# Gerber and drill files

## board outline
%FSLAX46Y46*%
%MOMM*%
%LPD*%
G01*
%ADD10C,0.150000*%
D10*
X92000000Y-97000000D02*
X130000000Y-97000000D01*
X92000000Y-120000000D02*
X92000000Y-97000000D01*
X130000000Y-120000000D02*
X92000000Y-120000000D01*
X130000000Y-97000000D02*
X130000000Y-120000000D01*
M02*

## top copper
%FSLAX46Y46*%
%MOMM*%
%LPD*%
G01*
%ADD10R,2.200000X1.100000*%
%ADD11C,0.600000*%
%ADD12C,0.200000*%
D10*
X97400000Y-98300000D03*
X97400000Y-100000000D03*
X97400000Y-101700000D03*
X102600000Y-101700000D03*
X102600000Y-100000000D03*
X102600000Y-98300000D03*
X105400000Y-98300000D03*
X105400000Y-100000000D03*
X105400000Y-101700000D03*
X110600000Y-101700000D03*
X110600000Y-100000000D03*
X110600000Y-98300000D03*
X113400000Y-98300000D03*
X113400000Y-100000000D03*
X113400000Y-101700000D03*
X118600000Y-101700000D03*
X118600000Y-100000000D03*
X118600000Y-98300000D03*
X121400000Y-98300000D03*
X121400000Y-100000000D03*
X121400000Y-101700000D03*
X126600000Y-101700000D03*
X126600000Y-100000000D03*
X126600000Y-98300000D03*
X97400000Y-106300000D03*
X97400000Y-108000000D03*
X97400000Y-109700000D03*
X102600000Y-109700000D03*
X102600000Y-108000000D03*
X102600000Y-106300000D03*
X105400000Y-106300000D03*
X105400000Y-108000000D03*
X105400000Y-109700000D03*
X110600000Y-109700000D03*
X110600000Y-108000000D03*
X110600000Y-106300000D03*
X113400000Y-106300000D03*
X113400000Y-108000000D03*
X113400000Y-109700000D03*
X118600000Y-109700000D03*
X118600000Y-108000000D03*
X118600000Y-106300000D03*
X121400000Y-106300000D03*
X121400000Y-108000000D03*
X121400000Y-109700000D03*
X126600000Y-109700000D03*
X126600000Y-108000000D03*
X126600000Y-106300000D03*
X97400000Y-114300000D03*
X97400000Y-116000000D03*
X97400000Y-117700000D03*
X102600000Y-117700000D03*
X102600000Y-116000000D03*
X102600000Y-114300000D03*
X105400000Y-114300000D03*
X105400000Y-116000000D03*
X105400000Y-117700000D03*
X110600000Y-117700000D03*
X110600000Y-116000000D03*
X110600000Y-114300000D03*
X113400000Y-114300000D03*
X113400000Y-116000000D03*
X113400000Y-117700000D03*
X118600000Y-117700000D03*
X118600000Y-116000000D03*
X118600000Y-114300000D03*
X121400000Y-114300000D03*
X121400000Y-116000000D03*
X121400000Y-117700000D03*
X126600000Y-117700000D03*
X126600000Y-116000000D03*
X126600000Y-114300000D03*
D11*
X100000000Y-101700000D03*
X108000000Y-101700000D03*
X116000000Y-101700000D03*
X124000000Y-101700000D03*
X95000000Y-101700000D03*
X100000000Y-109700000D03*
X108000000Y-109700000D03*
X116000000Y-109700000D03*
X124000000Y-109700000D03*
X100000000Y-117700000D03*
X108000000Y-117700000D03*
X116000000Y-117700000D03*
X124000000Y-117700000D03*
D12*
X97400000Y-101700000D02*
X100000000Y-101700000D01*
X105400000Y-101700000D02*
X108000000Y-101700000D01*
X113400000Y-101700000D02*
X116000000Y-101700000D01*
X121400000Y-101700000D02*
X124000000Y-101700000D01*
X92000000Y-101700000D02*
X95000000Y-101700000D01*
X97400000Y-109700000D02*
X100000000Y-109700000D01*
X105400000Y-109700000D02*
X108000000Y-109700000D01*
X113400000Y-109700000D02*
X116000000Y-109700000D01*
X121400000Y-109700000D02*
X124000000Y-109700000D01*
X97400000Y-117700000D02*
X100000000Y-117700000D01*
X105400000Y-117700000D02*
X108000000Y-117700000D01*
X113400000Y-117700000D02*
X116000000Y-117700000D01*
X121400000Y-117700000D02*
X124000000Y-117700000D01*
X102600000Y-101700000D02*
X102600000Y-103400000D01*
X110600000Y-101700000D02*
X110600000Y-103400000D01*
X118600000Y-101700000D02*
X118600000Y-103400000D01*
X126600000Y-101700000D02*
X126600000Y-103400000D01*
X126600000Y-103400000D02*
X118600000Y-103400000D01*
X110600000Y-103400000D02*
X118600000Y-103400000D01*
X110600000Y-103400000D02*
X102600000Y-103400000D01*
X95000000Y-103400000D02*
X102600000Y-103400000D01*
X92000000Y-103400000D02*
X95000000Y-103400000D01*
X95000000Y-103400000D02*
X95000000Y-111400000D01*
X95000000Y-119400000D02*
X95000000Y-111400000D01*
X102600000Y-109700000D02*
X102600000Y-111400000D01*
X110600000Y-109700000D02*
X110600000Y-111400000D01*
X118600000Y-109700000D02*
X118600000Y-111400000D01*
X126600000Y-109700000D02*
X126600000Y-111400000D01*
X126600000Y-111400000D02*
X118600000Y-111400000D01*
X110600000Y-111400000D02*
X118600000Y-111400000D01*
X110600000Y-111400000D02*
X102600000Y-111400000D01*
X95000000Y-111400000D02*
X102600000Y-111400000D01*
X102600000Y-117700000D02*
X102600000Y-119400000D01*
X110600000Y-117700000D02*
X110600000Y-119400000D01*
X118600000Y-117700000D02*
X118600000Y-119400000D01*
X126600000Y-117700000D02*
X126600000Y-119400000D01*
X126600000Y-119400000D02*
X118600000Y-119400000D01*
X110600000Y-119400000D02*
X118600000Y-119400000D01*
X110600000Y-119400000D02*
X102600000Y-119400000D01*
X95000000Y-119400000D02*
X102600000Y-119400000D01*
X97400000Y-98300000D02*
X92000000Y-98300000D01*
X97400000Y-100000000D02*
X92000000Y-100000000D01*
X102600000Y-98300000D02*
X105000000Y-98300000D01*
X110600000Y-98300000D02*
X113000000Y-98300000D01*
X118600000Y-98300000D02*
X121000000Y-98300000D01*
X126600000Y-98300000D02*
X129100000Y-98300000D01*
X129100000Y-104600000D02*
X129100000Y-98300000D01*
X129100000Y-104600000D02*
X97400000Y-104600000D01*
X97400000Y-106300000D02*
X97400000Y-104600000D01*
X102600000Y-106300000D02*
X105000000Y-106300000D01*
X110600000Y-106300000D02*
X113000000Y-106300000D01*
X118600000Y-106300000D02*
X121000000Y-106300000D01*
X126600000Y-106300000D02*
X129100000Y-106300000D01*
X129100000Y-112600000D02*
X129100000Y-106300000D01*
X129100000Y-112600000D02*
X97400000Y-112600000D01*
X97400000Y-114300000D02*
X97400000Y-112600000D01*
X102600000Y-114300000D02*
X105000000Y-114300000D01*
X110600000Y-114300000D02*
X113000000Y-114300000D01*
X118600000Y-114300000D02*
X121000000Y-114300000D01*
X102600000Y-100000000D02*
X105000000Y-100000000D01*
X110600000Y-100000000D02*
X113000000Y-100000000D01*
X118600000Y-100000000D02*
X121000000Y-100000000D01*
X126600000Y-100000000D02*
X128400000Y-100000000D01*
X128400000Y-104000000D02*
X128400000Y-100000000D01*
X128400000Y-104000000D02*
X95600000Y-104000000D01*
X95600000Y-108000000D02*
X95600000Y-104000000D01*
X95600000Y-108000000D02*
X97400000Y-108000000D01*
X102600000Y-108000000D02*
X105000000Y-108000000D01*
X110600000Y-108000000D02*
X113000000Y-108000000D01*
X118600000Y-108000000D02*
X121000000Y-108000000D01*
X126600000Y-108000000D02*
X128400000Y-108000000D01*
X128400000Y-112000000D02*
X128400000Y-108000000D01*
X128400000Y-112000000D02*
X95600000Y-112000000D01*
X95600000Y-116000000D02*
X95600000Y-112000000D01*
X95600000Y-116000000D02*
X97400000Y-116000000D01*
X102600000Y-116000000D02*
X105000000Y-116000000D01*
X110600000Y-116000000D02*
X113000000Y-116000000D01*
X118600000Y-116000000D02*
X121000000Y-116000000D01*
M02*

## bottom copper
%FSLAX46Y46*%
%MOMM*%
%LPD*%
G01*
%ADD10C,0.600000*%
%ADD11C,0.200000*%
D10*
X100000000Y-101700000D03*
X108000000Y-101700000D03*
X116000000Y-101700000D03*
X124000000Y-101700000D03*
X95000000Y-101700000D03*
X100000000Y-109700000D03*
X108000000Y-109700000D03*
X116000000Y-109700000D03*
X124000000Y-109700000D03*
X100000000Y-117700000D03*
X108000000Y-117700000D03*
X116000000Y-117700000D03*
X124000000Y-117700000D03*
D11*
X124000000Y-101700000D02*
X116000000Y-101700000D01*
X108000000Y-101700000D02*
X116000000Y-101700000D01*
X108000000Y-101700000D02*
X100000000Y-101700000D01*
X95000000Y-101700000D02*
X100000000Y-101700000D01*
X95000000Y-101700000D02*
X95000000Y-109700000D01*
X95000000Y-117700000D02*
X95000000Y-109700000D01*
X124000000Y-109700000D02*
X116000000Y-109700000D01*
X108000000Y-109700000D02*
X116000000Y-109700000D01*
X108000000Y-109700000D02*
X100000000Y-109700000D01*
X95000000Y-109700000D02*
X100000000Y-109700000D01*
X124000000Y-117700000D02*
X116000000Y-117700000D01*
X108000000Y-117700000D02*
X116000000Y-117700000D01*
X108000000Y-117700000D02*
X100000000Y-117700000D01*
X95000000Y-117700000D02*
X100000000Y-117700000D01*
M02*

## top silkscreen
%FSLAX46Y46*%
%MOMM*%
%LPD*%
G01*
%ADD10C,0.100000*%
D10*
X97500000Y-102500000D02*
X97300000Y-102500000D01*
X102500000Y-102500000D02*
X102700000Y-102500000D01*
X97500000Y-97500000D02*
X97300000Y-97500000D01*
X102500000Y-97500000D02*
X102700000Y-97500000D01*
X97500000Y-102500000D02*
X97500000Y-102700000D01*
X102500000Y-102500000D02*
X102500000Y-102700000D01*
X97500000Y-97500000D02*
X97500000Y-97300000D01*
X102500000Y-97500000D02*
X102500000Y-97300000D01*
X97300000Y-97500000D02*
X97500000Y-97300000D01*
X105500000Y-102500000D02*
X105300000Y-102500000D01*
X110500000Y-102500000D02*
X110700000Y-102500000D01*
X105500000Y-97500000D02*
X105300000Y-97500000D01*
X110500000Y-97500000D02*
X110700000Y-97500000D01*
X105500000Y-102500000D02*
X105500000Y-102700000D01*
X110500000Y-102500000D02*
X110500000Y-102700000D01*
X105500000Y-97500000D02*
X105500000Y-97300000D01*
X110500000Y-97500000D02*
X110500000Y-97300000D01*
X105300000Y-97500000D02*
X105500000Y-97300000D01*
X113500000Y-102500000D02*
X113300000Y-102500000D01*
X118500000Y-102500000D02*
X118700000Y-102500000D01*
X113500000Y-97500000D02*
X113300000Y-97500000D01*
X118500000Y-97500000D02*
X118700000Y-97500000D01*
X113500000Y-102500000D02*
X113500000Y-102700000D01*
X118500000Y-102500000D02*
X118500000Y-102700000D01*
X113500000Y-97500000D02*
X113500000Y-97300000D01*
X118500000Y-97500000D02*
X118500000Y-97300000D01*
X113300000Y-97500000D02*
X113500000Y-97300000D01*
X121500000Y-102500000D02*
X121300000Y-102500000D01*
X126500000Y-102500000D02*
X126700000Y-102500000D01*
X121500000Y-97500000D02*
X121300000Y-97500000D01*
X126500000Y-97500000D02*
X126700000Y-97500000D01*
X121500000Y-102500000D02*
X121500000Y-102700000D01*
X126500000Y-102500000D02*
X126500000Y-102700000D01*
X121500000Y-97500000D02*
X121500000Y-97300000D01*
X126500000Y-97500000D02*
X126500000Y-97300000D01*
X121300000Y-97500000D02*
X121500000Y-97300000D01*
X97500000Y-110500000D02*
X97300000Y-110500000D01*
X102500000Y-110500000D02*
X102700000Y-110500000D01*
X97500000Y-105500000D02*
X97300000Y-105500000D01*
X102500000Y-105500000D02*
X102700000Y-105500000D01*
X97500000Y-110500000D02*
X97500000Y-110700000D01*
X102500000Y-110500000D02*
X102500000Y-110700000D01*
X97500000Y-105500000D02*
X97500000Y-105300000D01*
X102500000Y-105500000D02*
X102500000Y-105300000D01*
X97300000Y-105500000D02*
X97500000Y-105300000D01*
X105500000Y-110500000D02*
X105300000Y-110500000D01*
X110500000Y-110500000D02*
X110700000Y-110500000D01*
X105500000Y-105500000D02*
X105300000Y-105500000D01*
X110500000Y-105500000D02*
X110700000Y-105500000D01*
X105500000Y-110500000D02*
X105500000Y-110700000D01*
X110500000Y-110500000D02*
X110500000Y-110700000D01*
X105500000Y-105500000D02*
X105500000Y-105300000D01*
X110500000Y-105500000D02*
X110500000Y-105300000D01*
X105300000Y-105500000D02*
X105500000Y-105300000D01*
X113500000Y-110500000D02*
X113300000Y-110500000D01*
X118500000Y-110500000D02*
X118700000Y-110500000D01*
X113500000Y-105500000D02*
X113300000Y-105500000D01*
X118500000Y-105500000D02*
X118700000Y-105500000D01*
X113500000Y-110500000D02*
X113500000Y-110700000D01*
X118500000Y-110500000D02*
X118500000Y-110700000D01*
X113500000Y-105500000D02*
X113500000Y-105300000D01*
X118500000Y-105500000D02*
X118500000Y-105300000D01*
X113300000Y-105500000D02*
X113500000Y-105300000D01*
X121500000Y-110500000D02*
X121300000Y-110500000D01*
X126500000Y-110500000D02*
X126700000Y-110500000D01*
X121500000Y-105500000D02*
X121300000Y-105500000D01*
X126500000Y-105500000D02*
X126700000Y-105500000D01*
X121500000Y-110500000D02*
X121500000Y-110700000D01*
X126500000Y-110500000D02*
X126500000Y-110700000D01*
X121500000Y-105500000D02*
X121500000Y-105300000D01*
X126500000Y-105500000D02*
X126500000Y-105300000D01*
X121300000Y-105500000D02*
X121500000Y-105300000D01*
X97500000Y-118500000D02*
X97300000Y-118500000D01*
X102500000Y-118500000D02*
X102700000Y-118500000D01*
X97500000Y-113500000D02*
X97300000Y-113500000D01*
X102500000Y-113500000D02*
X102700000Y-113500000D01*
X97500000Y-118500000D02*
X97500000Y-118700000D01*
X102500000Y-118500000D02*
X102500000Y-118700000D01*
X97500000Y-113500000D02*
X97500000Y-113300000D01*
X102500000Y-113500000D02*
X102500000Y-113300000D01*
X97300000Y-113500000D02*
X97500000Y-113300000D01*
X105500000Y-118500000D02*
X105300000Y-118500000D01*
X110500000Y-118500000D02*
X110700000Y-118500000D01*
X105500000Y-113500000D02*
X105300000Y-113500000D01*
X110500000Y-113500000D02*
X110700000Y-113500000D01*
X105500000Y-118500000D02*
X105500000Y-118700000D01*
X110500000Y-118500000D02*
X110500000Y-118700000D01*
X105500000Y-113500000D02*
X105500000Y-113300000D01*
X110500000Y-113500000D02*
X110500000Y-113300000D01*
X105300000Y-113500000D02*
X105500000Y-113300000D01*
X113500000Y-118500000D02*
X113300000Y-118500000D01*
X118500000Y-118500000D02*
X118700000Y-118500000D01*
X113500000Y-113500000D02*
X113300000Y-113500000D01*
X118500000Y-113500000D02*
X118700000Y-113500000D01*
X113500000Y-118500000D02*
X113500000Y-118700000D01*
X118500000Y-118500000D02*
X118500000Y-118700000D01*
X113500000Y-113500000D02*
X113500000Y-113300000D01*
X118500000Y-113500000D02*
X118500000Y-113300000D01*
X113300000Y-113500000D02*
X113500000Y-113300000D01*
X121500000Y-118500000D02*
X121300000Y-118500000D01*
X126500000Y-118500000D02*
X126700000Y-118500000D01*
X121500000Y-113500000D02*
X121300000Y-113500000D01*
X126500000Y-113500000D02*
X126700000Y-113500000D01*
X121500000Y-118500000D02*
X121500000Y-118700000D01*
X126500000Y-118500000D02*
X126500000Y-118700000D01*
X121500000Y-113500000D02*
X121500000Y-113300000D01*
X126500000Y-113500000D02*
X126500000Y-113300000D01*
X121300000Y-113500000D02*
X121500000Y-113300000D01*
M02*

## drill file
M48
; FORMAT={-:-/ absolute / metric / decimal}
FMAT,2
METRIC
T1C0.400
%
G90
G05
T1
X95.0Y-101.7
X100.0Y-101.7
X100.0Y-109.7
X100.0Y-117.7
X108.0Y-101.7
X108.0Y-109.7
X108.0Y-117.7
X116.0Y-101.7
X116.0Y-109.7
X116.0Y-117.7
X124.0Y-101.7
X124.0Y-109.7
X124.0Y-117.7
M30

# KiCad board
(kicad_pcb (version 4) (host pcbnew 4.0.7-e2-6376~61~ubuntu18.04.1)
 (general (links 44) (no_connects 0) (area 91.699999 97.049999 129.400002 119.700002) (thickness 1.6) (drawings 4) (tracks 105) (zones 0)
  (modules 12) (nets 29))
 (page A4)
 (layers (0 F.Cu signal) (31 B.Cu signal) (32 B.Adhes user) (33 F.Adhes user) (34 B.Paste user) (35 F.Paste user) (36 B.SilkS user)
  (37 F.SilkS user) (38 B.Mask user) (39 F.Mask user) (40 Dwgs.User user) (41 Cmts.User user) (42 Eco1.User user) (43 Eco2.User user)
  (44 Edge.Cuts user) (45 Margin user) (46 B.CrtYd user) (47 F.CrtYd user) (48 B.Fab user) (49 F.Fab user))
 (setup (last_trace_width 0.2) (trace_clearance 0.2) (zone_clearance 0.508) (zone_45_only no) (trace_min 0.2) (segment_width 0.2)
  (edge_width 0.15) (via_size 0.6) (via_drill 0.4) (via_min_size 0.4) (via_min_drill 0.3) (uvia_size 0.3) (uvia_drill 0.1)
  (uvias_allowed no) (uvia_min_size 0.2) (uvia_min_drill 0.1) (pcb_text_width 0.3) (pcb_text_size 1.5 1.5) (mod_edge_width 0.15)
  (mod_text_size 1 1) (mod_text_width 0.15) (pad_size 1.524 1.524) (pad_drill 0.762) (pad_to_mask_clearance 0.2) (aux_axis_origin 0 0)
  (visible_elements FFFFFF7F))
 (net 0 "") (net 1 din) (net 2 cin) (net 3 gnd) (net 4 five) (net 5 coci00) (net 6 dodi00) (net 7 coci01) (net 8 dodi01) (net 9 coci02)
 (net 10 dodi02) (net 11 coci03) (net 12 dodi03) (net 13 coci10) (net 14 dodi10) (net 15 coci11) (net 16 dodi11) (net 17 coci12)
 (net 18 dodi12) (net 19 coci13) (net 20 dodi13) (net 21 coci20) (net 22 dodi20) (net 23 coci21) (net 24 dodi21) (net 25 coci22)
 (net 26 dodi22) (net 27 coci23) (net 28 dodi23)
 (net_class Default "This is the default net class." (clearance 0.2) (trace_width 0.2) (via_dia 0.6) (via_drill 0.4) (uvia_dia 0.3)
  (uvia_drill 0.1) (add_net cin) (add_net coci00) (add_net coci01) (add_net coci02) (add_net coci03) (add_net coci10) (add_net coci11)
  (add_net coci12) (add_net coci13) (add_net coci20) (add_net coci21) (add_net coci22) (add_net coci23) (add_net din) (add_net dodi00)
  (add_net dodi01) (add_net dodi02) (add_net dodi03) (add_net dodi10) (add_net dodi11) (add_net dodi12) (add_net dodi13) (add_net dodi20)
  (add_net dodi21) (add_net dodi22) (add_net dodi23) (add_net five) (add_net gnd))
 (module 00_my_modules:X (layer F.Cu) (at 100 100)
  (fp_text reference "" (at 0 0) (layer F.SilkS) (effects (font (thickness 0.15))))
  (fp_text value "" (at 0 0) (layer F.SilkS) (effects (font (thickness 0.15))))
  (fp_line (start -2.5 2.5) (end -2.7 2.5) (layer F.SilkS) (width 0.1))
  (fp_line (start 2.5 2.5) (end 2.7 2.5) (layer F.SilkS) (width 0.1))
  (fp_line (start -2.5 -2.5) (end -2.7 -2.5) (layer F.SilkS) (width 0.1))
  (fp_line (start 2.5 -2.5) (end 2.7 -2.5) (layer F.SilkS) (width 0.1))
  (fp_line (start -2.5 2.5) (end -2.5 2.7) (layer F.SilkS) (width 0.1))
  (fp_line (start 2.5 2.5) (end 2.5 2.7) (layer F.SilkS) (width 0.1))
  (fp_line (start -2.5 -2.5) (end -2.5 -2.7) (layer F.SilkS) (width 0.1))
  (fp_line (start 2.5 -2.5) (end 2.5 -2.7) (layer F.SilkS) (width 0.1))
  (fp_line (start -2.7 -2.5) (end -2.5 -2.7) (layer F.SilkS) (width 0.1))
  (pad XX smd rect (at -2.6 -1.7) (size 2.2 1.1) (layers B.Mask))
  (pad DI smd rect (at -2.6 -1.7) (size 2.2 1.1) (layers F.Cu F.Paste F.Mask) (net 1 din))
  (pad CI smd rect (at -2.6 0) (size 2.2 1.1) (layers F.Cu F.Paste F.Mask) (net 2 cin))
  (pad GND smd rect (at -2.6 1.7) (size 2.2 1.1) (layers F.Cu F.Paste F.Mask) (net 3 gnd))
  (pad 5V smd rect (at 2.6 1.7) (size 2.2 1.1) (layers F.Cu F.Paste F.Mask) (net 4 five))
  (pad CO smd rect (at 2.6 0) (size 2.2 1.1) (layers F.Cu F.Paste F.Mask) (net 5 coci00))
  (pad DO smd rect (at 2.6 -1.7) (size 2.2 1.1) (layers F.Cu F.Paste F.Mask) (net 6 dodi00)))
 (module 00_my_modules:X (layer F.Cu) (at 108 100)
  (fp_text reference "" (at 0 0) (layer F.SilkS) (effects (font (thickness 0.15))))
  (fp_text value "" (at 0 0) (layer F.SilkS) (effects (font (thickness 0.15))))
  (fp_line (start -2.5 2.5) (end -2.7 2.5) (layer F.SilkS) (width 0.1))
  (fp_line (start 2.5 2.5) (end 2.7 2.5) (layer F.SilkS) (width 0.1))
  (fp_line (start -2.5 -2.5) (end -2.7 -2.5) (layer F.SilkS) (width 0.1))
  (fp_line (start 2.5 -2.5) (end 2.7 -2.5) (layer F.SilkS) (width 0.1))
  (fp_line (start -2.5 2.5) (end -2.5 2.7) (layer F.SilkS) (width 0.1))
  (fp_line (start 2.5 2.5) (end 2.5 2.7) (layer F.SilkS) (width 0.1))
  (fp_line (start -2.5 -2.5) (end -2.5 -2.7) (layer F.SilkS) (width 0.1))
  (fp_line (start 2.5 -2.5) (end 2.5 -2.7) (layer F.SilkS) (width 0.1))
  (fp_line (start -2.7 -2.5) (end -2.5 -2.7) (layer F.SilkS) (width 0.1))
  (pad DI smd rect (at -2.6 -1.7) (size 2.2 1.1) (layers F.Cu F.Paste F.Mask) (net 6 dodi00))
  (pad CI smd rect (at -2.6 0) (size 2.2 1.1) (layers F.Cu F.Paste F.Mask) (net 5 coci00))
  (pad GND smd rect (at -2.6 1.7) (size 2.2 1.1) (layers F.Cu F.Paste F.Mask) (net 3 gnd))
  (pad 5V smd rect (at 2.6 1.7) (size 2.2 1.1) (layers F.Cu F.Paste F.Mask) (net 4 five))
  (pad CO smd rect (at 2.6 0) (size 2.2 1.1) (layers F.Cu F.Paste F.Mask) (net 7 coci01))
  (pad DO smd rect (at 2.6 -1.7) (size 2.2 1.1) (layers F.Cu F.Paste F.Mask) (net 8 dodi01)))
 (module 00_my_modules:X (layer F.Cu) (at 116 100)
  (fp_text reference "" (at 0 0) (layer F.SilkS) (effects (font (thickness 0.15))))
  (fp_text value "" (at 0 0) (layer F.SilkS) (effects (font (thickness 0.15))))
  (fp_line (start -2.5 2.5) (end -2.7 2.5) (layer F.SilkS) (width 0.1))
  (fp_line (start 2.5 2.5) (end 2.7 2.5) (layer F.SilkS) (width 0.1))
  (fp_line (start -2.5 -2.5) (end -2.7 -2.5) (layer F.SilkS) (width 0.1))
  (fp_line (start 2.5 -2.5) (end 2.7 -2.5) (layer F.SilkS) (width 0.1))
  (fp_line (start -2.5 2.5) (end -2.5 2.7) (layer F.SilkS) (width 0.1))
  (fp_line (start 2.5 2.5) (end 2.5 2.7) (layer F.SilkS) (width 0.1))
  (fp_line (start -2.5 -2.5) (end -2.5 -2.7) (layer F.SilkS) (width 0.1))
  (fp_line (start 2.5 -2.5) (end 2.5 -2.7) (layer F.SilkS) (width 0.1))
  (fp_line (start -2.7 -2.5) (end -2.5 -2.7) (layer F.SilkS) (width 0.1))
  (pad DI smd rect (at -2.6 -1.7) (size 2.2 1.1) (layers F.Cu F.Paste F.Mask) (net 8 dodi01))
  (pad CI smd rect (at -2.6 0) (size 2.2 1.1) (layers F.Cu F.Paste F.Mask) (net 7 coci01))
  (pad GND smd rect (at -2.6 1.7) (size 2.2 1.1) (layers F.Cu F.Paste F.Mask) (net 3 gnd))
  (pad 5V smd rect (at 2.6 1.7) (size 2.2 1.1) (layers F.Cu F.Paste F.Mask) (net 4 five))
  (pad CO smd rect (at 2.6 0) (size 2.2 1.1) (layers F.Cu F.Paste F.Mask) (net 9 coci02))
  (pad DO smd rect (at 2.6 -1.7) (size 2.2 1.1) (layers F.Cu F.Paste F.Mask) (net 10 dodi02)))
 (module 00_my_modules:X (layer F.Cu) (at 124 100)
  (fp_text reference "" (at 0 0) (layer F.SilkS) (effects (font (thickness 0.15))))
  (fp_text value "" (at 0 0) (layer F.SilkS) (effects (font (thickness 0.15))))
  (fp_line (start -2.5 2.5) (end -2.7 2.5) (layer F.SilkS) (width 0.1))
  (fp_line (start 2.5 2.5) (end 2.7 2.5) (layer F.SilkS) (width 0.1))
  (fp_line (start -2.5 -2.5) (end -2.7 -2.5) (layer F.SilkS) (width 0.1))
  (fp_line (start 2.5 -2.5) (end 2.7 -2.5) (layer F.SilkS) (width 0.1))
  (fp_line (start -2.5 2.5) (end -2.5 2.7) (layer F.SilkS) (width 0.1))
  (fp_line (start 2.5 2.5) (end 2.5 2.7) (layer F.SilkS) (width 0.1))
  (fp_line (start -2.5 -2.5) (end -2.5 -2.7) (layer F.SilkS) (width 0.1))
  (fp_line (start 2.5 -2.5) (end 2.5 -2.7) (layer F.SilkS) (width 0.1))
  (fp_line (start -2.7 -2.5) (end -2.5 -2.7) (layer F.SilkS) (width 0.1))
  (pad DI smd rect (at -2.6 -1.7) (size 2.2 1.1) (layers F.Cu F.Paste F.Mask) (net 10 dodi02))
  (pad CI smd rect (at -2.6 0) (size 2.2 1.1) (layers F.Cu F.Paste F.Mask) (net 9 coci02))
  (pad GND smd rect (at -2.6 1.7) (size 2.2 1.1) (layers F.Cu F.Paste F.Mask) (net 3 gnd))
  (pad 5V smd rect (at 2.6 1.7) (size 2.2 1.1) (layers F.Cu F.Paste F.Mask) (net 4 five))
  (pad CO smd rect (at 2.6 0) (size 2.2 1.1) (layers F.Cu F.Paste F.Mask) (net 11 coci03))
  (pad DO smd rect (at 2.6 -1.7) (size 2.2 1.1) (layers F.Cu F.Paste F.Mask) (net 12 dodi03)))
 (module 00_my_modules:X (layer F.Cu) (at 100 108)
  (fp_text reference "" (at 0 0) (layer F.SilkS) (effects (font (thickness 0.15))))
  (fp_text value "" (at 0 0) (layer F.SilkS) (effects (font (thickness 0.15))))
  (fp_line (start -2.5 2.5) (end -2.7 2.5) (layer F.SilkS) (width 0.1))
  (fp_line (start 2.5 2.5) (end 2.7 2.5) (layer F.SilkS) (width 0.1))
  (fp_line (start -2.5 -2.5) (end -2.7 -2.5) (layer F.SilkS) (width 0.1))
  (fp_line (start 2.5 -2.5) (end 2.7 -2.5) (layer F.SilkS) (width 0.1))
  (fp_line (start -2.5 2.5) (end -2.5 2.7) (layer F.SilkS) (width 0.1))
  (fp_line (start 2.5 2.5) (end 2.5 2.7) (layer F.SilkS) (width 0.1))
  (fp_line (start -2.5 -2.5) (end -2.5 -2.7) (layer F.SilkS) (width 0.1))
  (fp_line (start 2.5 -2.5) (end 2.5 -2.7) (layer F.SilkS) (width 0.1))
  (fp_line (start -2.7 -2.5) (end -2.5 -2.7) (layer F.SilkS) (width 0.1))
  (pad DI smd rect (at -2.6 -1.7) (size 2.2 1.1) (layers F.Cu F.Paste F.Mask) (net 12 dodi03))
  (pad CI smd rect (at -2.6 0) (size 2.2 1.1) (layers F.Cu F.Paste F.Mask) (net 11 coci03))
  (pad GND smd rect (at -2.6 1.7) (size 2.2 1.1) (layers F.Cu F.Paste F.Mask) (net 3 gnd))
  (pad 5V smd rect (at 2.6 1.7) (size 2.2 1.1) (layers F.Cu F.Paste F.Mask) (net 4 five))
  (pad CO smd rect (at 2.6 0) (size 2.2 1.1) (layers F.Cu F.Paste F.Mask) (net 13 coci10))
  (pad DO smd rect (at 2.6 -1.7) (size 2.2 1.1) (layers F.Cu F.Paste F.Mask) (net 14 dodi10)))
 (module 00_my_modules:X (layer F.Cu) (at 108 108)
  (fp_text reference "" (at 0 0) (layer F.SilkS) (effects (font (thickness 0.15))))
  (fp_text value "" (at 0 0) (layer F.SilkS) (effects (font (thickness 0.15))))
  (fp_line (start -2.5 2.5) (end -2.7 2.5) (layer F.SilkS) (width 0.1))
  (fp_line (start 2.5 2.5) (end 2.7 2.5) (layer F.SilkS) (width 0.1))
  (fp_line (start -2.5 -2.5) (end -2.7 -2.5) (layer F.SilkS) (width 0.1))
  (fp_line (start 2.5 -2.5) (end 2.7 -2.5) (layer F.SilkS) (width 0.1))
  (fp_line (start -2.5 2.5) (end -2.5 2.7) (layer F.SilkS) (width 0.1))
  (fp_line (start 2.5 2.5) (end 2.5 2.7) (layer F.SilkS) (width 0.1))
  (fp_line (start -2.5 -2.5) (end -2.5 -2.7) (layer F.SilkS) (width 0.1))
  (fp_line (start 2.5 -2.5) (end 2.5 -2.7) (layer F.SilkS) (width 0.1))
  (fp_line (start -2.7 -2.5) (end -2.5 -2.7) (layer F.SilkS) (width 0.1))
  (pad DI smd rect (at -2.6 -1.7) (size 2.2 1.1) (layers F.Cu F.Paste F.Mask) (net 14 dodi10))
  (pad CI smd rect (at -2.6 0) (size 2.2 1.1) (layers F.Cu F.Paste F.Mask) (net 13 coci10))
  (pad GND smd rect (at -2.6 1.7) (size 2.2 1.1) (layers F.Cu F.Paste F.Mask) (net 3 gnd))
  (pad 5V smd rect (at 2.6 1.7) (size 2.2 1.1) (layers F.Cu F.Paste F.Mask) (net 4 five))
  (pad CO smd rect (at 2.6 0) (size 2.2 1.1) (layers F.Cu F.Paste F.Mask) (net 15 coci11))
  (pad DO smd rect (at 2.6 -1.7) (size 2.2 1.1) (layers F.Cu F.Paste F.Mask) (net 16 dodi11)))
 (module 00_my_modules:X (layer F.Cu) (at 116 108)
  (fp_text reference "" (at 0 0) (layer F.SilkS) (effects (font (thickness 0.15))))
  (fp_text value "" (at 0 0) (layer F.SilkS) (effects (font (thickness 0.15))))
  (fp_line (start -2.5 2.5) (end -2.7 2.5) (layer F.SilkS) (width 0.1))
  (fp_line (start 2.5 2.5) (end 2.7 2.5) (layer F.SilkS) (width 0.1))
  (fp_line (start -2.5 -2.5) (end -2.7 -2.5) (layer F.SilkS) (width 0.1))
  (fp_line (start 2.5 -2.5) (end 2.7 -2.5) (layer F.SilkS) (width 0.1))
  (fp_line (start -2.5 2.5) (end -2.5 2.7) (layer F.SilkS) (width 0.1))
  (fp_line (start 2.5 2.5) (end 2.5 2.7) (layer F.SilkS) (width 0.1))
  (fp_line (start -2.5 -2.5) (end -2.5 -2.7) (layer F.SilkS) (width 0.1))
  (fp_line (start 2.5 -2.5) (end 2.5 -2.7) (layer F.SilkS) (width 0.1))
  (fp_line (start -2.7 -2.5) (end -2.5 -2.7) (layer F.SilkS) (width 0.1))
  (pad DI smd rect (at -2.6 -1.7) (size 2.2 1.1) (layers F.Cu F.Paste F.Mask) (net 16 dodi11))
  (pad CI smd rect (at -2.6 0) (size 2.2 1.1) (layers F.Cu F.Paste F.Mask) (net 15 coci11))
  (pad GND smd rect (at -2.6 1.7) (size 2.2 1.1) (layers F.Cu F.Paste F.Mask) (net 3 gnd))
  (pad 5V smd rect (at 2.6 1.7) (size 2.2 1.1) (layers F.Cu F.Paste F.Mask) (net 4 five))
  (pad CO smd rect (at 2.6 0) (size 2.2 1.1) (layers F.Cu F.Paste F.Mask) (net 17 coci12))
  (pad DO smd rect (at 2.6 -1.7) (size 2.2 1.1) (layers F.Cu F.Paste F.Mask) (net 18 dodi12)))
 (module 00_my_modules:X (layer F.Cu) (at 124 108)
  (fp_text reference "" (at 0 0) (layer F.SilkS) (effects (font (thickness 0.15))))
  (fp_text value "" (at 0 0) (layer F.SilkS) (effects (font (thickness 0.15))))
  (fp_line (start -2.5 2.5) (end -2.7 2.5) (layer F.SilkS) (width 0.1))
  (fp_line (start 2.5 2.5) (end 2.7 2.5) (layer F.SilkS) (width 0.1))
  (fp_line (start -2.5 -2.5) (end -2.7 -2.5) (layer F.SilkS) (width 0.1))
  (fp_line (start 2.5 -2.5) (end 2.7 -2.5) (layer F.SilkS) (width 0.1))
  (fp_line (start -2.5 2.5) (end -2.5 2.7) (layer F.SilkS) (width 0.1))
  (fp_line (start 2.5 2.5) (end 2.5 2.7) (layer F.SilkS) (width 0.1))
  (fp_line (start -2.5 -2.5) (end -2.5 -2.7) (layer F.SilkS) (width 0.1))
  (fp_line (start 2.5 -2.5) (end 2.5 -2.7) (layer F.SilkS) (width 0.1))
  (fp_line (start -2.7 -2.5) (end -2.5 -2.7) (layer F.SilkS) (width 0.1))
  (pad DI smd rect (at -2.6 -1.7) (size 2.2 1.1) (layers F.Cu F.Paste F.Mask) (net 18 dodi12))
  (pad CI smd rect (at -2.6 0) (size 2.2 1.1) (layers F.Cu F.Paste F.Mask) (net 17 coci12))
  (pad GND smd rect (at -2.6 1.7) (size 2.2 1.1) (layers F.Cu F.Paste F.Mask) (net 3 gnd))
  (pad 5V smd rect (at 2.6 1.7) (size 2.2 1.1) (layers F.Cu F.Paste F.Mask) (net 4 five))
  (pad CO smd rect (at 2.6 0) (size 2.2 1.1) (layers F.Cu F.Paste F.Mask) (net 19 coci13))
  (pad DO smd rect (at 2.6 -1.7) (size 2.2 1.1) (layers F.Cu F.Paste F.Mask) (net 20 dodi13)))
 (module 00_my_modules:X (layer F.Cu) (at 100 116)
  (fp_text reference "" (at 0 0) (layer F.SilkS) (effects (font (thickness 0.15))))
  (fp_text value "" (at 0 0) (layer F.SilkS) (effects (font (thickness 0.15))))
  (fp_line (start -2.5 2.5) (end -2.7 2.5) (layer F.SilkS) (width 0.1))
  (fp_line (start 2.5 2.5) (end 2.7 2.5) (layer F.SilkS) (width 0.1))
  (fp_line (start -2.5 -2.5) (end -2.7 -2.5) (layer F.SilkS) (width 0.1))
  (fp_line (start 2.5 -2.5) (end 2.7 -2.5) (layer F.SilkS) (width 0.1))
  (fp_line (start -2.5 2.5) (end -2.5 2.7) (layer F.SilkS) (width 0.1))
  (fp_line (start 2.5 2.5) (end 2.5 2.7) (layer F.SilkS) (width 0.1))
  (fp_line (start -2.5 -2.5) (end -2.5 -2.7) (layer F.SilkS) (width 0.1))
  (fp_line (start 2.5 -2.5) (end 2.5 -2.7) (layer F.SilkS) (width 0.1))
  (fp_line (start -2.7 -2.5) (end -2.5 -2.7) (layer F.SilkS) (width 0.1))
  (pad DI smd rect (at -2.6 -1.7) (size 2.2 1.1) (layers F.Cu F.Paste F.Mask) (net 20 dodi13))
  (pad CI smd rect (at -2.6 0) (size 2.2 1.1) (layers F.Cu F.Paste F.Mask) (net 19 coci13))
  (pad GND smd rect (at -2.6 1.7) (size 2.2 1.1) (layers F.Cu F.Paste F.Mask) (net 3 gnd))
  (pad 5V smd rect (at 2.6 1.7) (size 2.2 1.1) (layers F.Cu F.Paste F.Mask) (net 4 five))
  (pad CO smd rect (at 2.6 0) (size 2.2 1.1) (layers F.Cu F.Paste F.Mask) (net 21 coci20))
  (pad DO smd rect (at 2.6 -1.7) (size 2.2 1.1) (layers F.Cu F.Paste F.Mask) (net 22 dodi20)))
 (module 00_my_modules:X (layer F.Cu) (at 108 116)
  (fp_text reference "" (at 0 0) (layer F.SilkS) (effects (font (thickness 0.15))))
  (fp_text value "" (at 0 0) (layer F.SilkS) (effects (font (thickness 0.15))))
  (fp_line (start -2.5 2.5) (end -2.7 2.5) (layer F.SilkS) (width 0.1))
  (fp_line (start 2.5 2.5) (end 2.7 2.5) (layer F.SilkS) (width 0.1))
  (fp_line (start -2.5 -2.5) (end -2.7 -2.5) (layer F.SilkS) (width 0.1))
  (fp_line (start 2.5 -2.5) (end 2.7 -2.5) (layer F.SilkS) (width 0.1))
  (fp_line (start -2.5 2.5) (end -2.5 2.7) (layer F.SilkS) (width 0.1))
  (fp_line (start 2.5 2.5) (end 2.5 2.7) (layer F.SilkS) (width 0.1))
  (fp_line (start -2.5 -2.5) (end -2.5 -2.7) (layer F.SilkS) (width 0.1))
  (fp_line (start 2.5 -2.5) (end 2.5 -2.7) (layer F.SilkS) (width 0.1))
  (fp_line (start -2.7 -2.5) (end -2.5 -2.7) (layer F.SilkS) (width 0.1))
  (pad DI smd rect (at -2.6 -1.7) (size 2.2 1.1) (layers F.Cu F.Paste F.Mask) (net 22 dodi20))
  (pad CI smd rect (at -2.6 0) (size 2.2 1.1) (layers F.Cu F.Paste F.Mask) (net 21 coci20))
  (pad GND smd rect (at -2.6 1.7) (size 2.2 1.1) (layers F.Cu F.Paste F.Mask) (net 3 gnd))
  (pad 5V smd rect (at 2.6 1.7) (size 2.2 1.1) (layers F.Cu F.Paste F.Mask) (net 4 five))
  (pad CO smd rect (at 2.6 0) (size 2.2 1.1) (layers F.Cu F.Paste F.Mask) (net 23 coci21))
  (pad DO smd rect (at 2.6 -1.7) (size 2.2 1.1) (layers F.Cu F.Paste F.Mask) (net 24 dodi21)))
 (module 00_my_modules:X (layer F.Cu) (at 116 116)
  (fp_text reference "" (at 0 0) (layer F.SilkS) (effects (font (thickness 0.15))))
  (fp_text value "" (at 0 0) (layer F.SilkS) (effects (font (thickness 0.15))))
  (fp_line (start -2.5 2.5) (end -2.7 2.5) (layer F.SilkS) (width 0.1))
  (fp_line (start 2.5 2.5) (end 2.7 2.5) (layer F.SilkS) (width 0.1))
  (fp_line (start -2.5 -2.5) (end -2.7 -2.5) (layer F.SilkS) (width 0.1))
  (fp_line (start 2.5 -2.5) (end 2.7 -2.5) (layer F.SilkS) (width 0.1))
  (fp_line (start -2.5 2.5) (end -2.5 2.7) (layer F.SilkS) (width 0.1))
  (fp_line (start 2.5 2.5) (end 2.5 2.7) (layer F.SilkS) (width 0.1))
  (fp_line (start -2.5 -2.5) (end -2.5 -2.7) (layer F.SilkS) (width 0.1))
  (fp_line (start 2.5 -2.5) (end 2.5 -2.7) (layer F.SilkS) (width 0.1))
  (fp_line (start -2.7 -2.5) (end -2.5 -2.7) (layer F.SilkS) (width 0.1))
  (pad DI smd rect (at -2.6 -1.7) (size 2.2 1.1) (layers F.Cu F.Paste F.Mask) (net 24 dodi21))
  (pad CI smd rect (at -2.6 0) (size 2.2 1.1) (layers F.Cu F.Paste F.Mask) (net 23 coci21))
  (pad GND smd rect (at -2.6 1.7) (size 2.2 1.1) (layers F.Cu F.Paste F.Mask) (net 3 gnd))
  (pad 5V smd rect (at 2.6 1.7) (size 2.2 1.1) (layers F.Cu F.Paste F.Mask) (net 4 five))
  (pad CO smd rect (at 2.6 0) (size 2.2 1.1) (layers F.Cu F.Paste F.Mask) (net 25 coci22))
  (pad DO smd rect (at 2.6 -1.7) (size 2.2 1.1) (layers F.Cu F.Paste F.Mask) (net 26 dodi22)))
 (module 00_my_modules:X (layer F.Cu) (at 124 116)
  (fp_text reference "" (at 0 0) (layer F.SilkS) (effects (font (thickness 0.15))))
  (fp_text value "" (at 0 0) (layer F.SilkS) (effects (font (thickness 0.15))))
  (fp_line (start -2.5 2.5) (end -2.7 2.5) (layer F.SilkS) (width 0.1))
  (fp_line (start 2.5 2.5) (end 2.7 2.5) (layer F.SilkS) (width 0.1))
  (fp_line (start -2.5 -2.5) (end -2.7 -2.5) (layer F.SilkS) (width 0.1))
  (fp_line (start 2.5 -2.5) (end 2.7 -2.5) (layer F.SilkS) (width 0.1))
  (fp_line (start -2.5 2.5) (end -2.5 2.7) (layer F.SilkS) (width 0.1))
  (fp_line (start 2.5 2.5) (end 2.5 2.7) (layer F.SilkS) (width 0.1))
  (fp_line (start -2.5 -2.5) (end -2.5 -2.7) (layer F.SilkS) (width 0.1))
  (fp_line (start 2.5 -2.5) (end 2.5 -2.7) (layer F.SilkS) (width 0.1))
  (fp_line (start -2.7 -2.5) (end -2.5 -2.7) (layer F.SilkS) (width 0.1))
  (pad DI smd rect (at -2.6 -1.7) (size 2.2 1.1) (layers F.Cu F.Paste F.Mask) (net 26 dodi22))
  (pad CI smd rect (at -2.6 0) (size 2.2 1.1) (layers F.Cu F.Paste F.Mask) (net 25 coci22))
  (pad GND smd rect (at -2.6 1.7) (size 2.2 1.1) (layers F.Cu F.Paste F.Mask) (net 3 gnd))
  (pad 5V smd rect (at 2.6 1.7) (size 2.2 1.1) (layers F.Cu F.Paste F.Mask) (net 4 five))
  (pad CO smd rect (at 2.6 0) (size 2.2 1.1) (layers F.Cu F.Paste F.Mask) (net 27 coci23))
  (pad DO smd rect (at 2.6 -1.7) (size 2.2 1.1) (layers F.Cu F.Paste F.Mask) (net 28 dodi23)))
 (gr_line (start 92 97) (end 130 97) (angle 90) (layer Edge.Cuts) (width 0.15))
 (gr_line (start 92 120) (end 92 97) (angle 90) (layer Edge.Cuts) (width 0.15))
 (gr_line (start 130 120) (end 92 120) (angle 90) (layer Edge.Cuts) (width 0.15))
 (gr_line (start 130 97) (end 130 120) (angle 90) (layer Edge.Cuts) (width 0.15))
 (segment (start 97.4 101.7) (end 100 101.7) (width 0.2) (layer F.Cu) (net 3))
 (via (at 100 101.7) (size 0.6) (drill 0.4) (layers F.Cu B.Cu) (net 3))
 (segment (start 105.4 101.7) (end 108 101.7) (width 0.2) (layer F.Cu) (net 3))
 (via (at 108 101.7) (size 0.6) (drill 0.4) (layers F.Cu B.Cu) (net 3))
 (segment (start 113.4 101.7) (end 116 101.7) (width 0.2) (layer F.Cu) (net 3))
 (via (at 116 101.7) (size 0.6) (drill 0.4) (layers F.Cu B.Cu) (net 3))
 (segment (start 121.4 101.7) (end 124 101.7) (width 0.2) (layer F.Cu) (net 3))
 (via (at 124 101.7) (size 0.6) (drill 0.4) (layers F.Cu B.Cu) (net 3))
 (segment (start 124 101.7) (end 116 101.7) (width 0.2) (layer B.Cu) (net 3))
 (segment (start 108 101.7) (end 116 101.7) (width 0.2) (layer B.Cu) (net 3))
 (segment (start 108 101.7) (end 100 101.7) (width 0.2) (layer B.Cu) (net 3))
 (segment (start 95 101.7) (end 100 101.7) (width 0.2) (layer B.Cu) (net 3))
 (via (at 95 101.7) (size 0.6) (drill 0.4) (layers F.Cu B.Cu) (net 3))
 (segment (start 92 101.7) (end 95 101.7) (width 0.2) (layer F.Cu) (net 3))
 (segment (start 95 101.7) (end 95 109.7) (width 0.2) (layer B.Cu) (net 3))
 (segment (start 95 117.7) (end 95 109.7) (width 0.2) (layer B.Cu) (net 3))
 (segment (start 97.4 109.7) (end 100 109.7) (width 0.2) (layer F.Cu) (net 3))
 (via (at 100 109.7) (size 0.6) (drill 0.4) (layers F.Cu B.Cu) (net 3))
 (segment (start 105.4 109.7) (end 108 109.7) (width 0.2) (layer F.Cu) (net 3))
 (via (at 108 109.7) (size 0.6) (drill 0.4) (layers F.Cu B.Cu) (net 3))
 (segment (start 113.4 109.7) (end 116 109.7) (width 0.2) (layer F.Cu) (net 3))
 (via (at 116 109.7) (size 0.6) (drill 0.4) (layers F.Cu B.Cu) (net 3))
 (segment (start 121.4 109.7) (end 124 109.7) (width 0.2) (layer F.Cu) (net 3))
 (via (at 124 109.7) (size 0.6) (drill 0.4) (layers F.Cu B.Cu) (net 3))
 (segment (start 124 109.7) (end 116 109.7) (width 0.2) (layer B.Cu) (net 3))
 (segment (start 108 109.7) (end 116 109.7) (width 0.2) (layer B.Cu) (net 3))
 (segment (start 108 109.7) (end 100 109.7) (width 0.2) (layer B.Cu) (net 3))
 (segment (start 95 109.7) (end 100 109.7) (width 0.2) (layer B.Cu) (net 3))
 (segment (start 97.4 117.7) (end 100 117.7) (width 0.2) (layer F.Cu) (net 3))
 (via (at 100 117.7) (size 0.6) (drill 0.4) (layers F.Cu B.Cu) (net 3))
 (segment (start 105.4 117.7) (end 108 117.7) (width 0.2) (layer F.Cu) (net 3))
 (via (at 108 117.7) (size 0.6) (drill 0.4) (layers F.Cu B.Cu) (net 3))
 (segment (start 113.4 117.7) (end 116 117.7) (width 0.2) (layer F.Cu) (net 3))
 (via (at 116 117.7) (size 0.6) (drill 0.4) (layers F.Cu B.Cu) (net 3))
 (segment (start 121.4 117.7) (end 124 117.7) (width 0.2) (layer F.Cu) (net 3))
 (via (at 124 117.7) (size 0.6) (drill 0.4) (layers F.Cu B.Cu) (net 3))
 (segment (start 124 117.7) (end 116 117.7) (width 0.2) (layer B.Cu) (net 3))
 (segment (start 108 117.7) (end 116 117.7) (width 0.2) (layer B.Cu) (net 3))
 (segment (start 108 117.7) (end 100 117.7) (width 0.2) (layer B.Cu) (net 3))
 (segment (start 95 117.7) (end 100 117.7) (width 0.2) (layer B.Cu) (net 3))
 (segment (start 102.6 101.7) (end 102.6 103.4) (width 0.2) (layer F.Cu) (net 4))
 (segment (start 110.6 101.7) (end 110.6 103.4) (width 0.2) (layer F.Cu) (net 4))
 (segment (start 118.6 101.7) (end 118.6 103.4) (width 0.2) (layer F.Cu) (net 4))
 (segment (start 126.6 101.7) (end 126.6 103.4) (width 0.2) (layer F.Cu) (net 4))
 (segment (start 126.6 103.4) (end 118.6 103.4) (width 0.2) (layer F.Cu) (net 4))
 (segment (start 110.6 103.4) (end 118.6 103.4) (width 0.2) (layer F.Cu) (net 4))
 (segment (start 110.6 103.4) (end 102.6 103.4) (width 0.2) (layer F.Cu) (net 4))
 (segment (start 95 103.4) (end 102.6 103.4) (width 0.2) (layer F.Cu) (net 4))
 (segment (start 92 103.4) (end 95 103.4) (width 0.2) (layer F.Cu) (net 4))
 (segment (start 95 103.4) (end 95 111.4) (width 0.2) (layer F.Cu) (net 4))
 (segment (start 95 119.4) (end 95 111.4) (width 0.2) (layer F.Cu) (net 4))
 (segment (start 102.6 109.7) (end 102.6 111.4) (width 0.2) (layer F.Cu) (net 4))
 (segment (start 110.6 109.7) (end 110.6 111.4) (width 0.2) (layer F.Cu) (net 4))
 (segment (start 118.6 109.7) (end 118.6 111.4) (width 0.2) (layer F.Cu) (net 4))
 (segment (start 126.6 109.7) (end 126.6 111.4) (width 0.2) (layer F.Cu) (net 4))
 (segment (start 126.6 111.4) (end 118.6 111.4) (width 0.2) (layer F.Cu) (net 4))
 (segment (start 110.6 111.4) (end 118.6 111.4) (width 0.2) (layer F.Cu) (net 4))
 (segment (start 110.6 111.4) (end 102.6 111.4) (width 0.2) (layer F.Cu) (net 4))
 (segment (start 95 111.4) (end 102.6 111.4) (width 0.2) (layer F.Cu) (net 4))
 (segment (start 102.6 117.7) (end 102.6 119.4) (width 0.2) (layer F.Cu) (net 4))
 (segment (start 110.6 117.7) (end 110.6 119.4) (width 0.2) (layer F.Cu) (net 4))
 (segment (start 118.6 117.7) (end 118.6 119.4) (width 0.2) (layer F.Cu) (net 4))
 (segment (start 126.6 117.7) (end 126.6 119.4) (width 0.2) (layer F.Cu) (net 4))
 (segment (start 126.6 119.4) (end 118.6 119.4) (width 0.2) (layer F.Cu) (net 4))
 (segment (start 110.6 119.4) (end 118.6 119.4) (width 0.2) (layer F.Cu) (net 4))
 (segment (start 110.6 119.4) (end 102.6 119.4) (width 0.2) (layer F.Cu) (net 4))
 (segment (start 95 119.4) (end 102.6 119.4) (width 0.2) (layer F.Cu) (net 4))
 (segment (start 97.4 98.3) (end 92 98.3) (width 0.2) (layer F.Cu) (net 1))
 (segment (start 97.4 100) (end 92 100) (width 0.2) (layer F.Cu) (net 2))
 (segment (start 102.6 98.3) (end 105 98.3) (width 0.2) (layer F.Cu) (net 6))
 (segment (start 110.6 98.3) (end 113 98.3) (width 0.2) (layer F.Cu) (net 8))
 (segment (start 118.6 98.3) (end 121 98.3) (width 0.2) (layer F.Cu) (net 10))
 (segment (start 126.6 98.3) (end 129.1 98.3) (width 0.2) (layer F.Cu) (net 12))
 (segment (start 129.1 104.6) (end 129.1 98.3) (width 0.2) (layer F.Cu) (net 12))
 (segment (start 129.1 104.6) (end 97.4 104.6) (width 0.2) (layer F.Cu) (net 12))
 (segment (start 97.4 106.3) (end 97.4 104.6) (width 0.2) (layer F.Cu) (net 12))
 (segment (start 102.6 106.3) (end 105 106.3) (width 0.2) (layer F.Cu) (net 14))
 (segment (start 110.6 106.3) (end 113 106.3) (width 0.2) (layer F.Cu) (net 16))
 (segment (start 118.6 106.3) (end 121 106.3) (width 0.2) (layer F.Cu) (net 18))
 (segment (start 126.6 106.3) (end 129.1 106.3) (width 0.2) (layer F.Cu) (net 20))
 (segment (start 129.1 112.6) (end 129.1 106.3) (width 0.2) (layer F.Cu) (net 20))
 (segment (start 129.1 112.6) (end 97.4 112.6) (width 0.2) (layer F.Cu) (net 20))
 (segment (start 97.4 114.3) (end 97.4 112.6) (width 0.2) (layer F.Cu) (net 20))
 (segment (start 102.6 114.3) (end 105 114.3) (width 0.2) (layer F.Cu) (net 22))
 (segment (start 110.6 114.3) (end 113 114.3) (width 0.2) (layer F.Cu) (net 24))
 (segment (start 118.6 114.3) (end 121 114.3) (width 0.2) (layer F.Cu) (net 26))
 (segment (start 102.6 100) (end 105 100) (width 0.2) (layer F.Cu) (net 5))
 (segment (start 110.6 100) (end 113 100) (width 0.2) (layer F.Cu) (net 7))
 (segment (start 118.6 100) (end 121 100) (width 0.2) (layer F.Cu) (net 9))
 (segment (start 126.6 100) (end 128.4 100) (width 0.2) (layer F.Cu) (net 11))
 (segment (start 128.4 104) (end 128.4 100) (width 0.2) (layer F.Cu) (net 11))
 (segment (start 128.4 104) (end 95.6 104) (width 0.2) (layer F.Cu) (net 11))
 (segment (start 95.6 108) (end 95.6 104) (width 0.2) (layer F.Cu) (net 11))
 (segment (start 95.6 108) (end 97.4 108) (width 0.2) (layer F.Cu) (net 11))
 (segment (start 102.6 108) (end 105 108) (width 0.2) (layer F.Cu) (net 13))
 (segment (start 110.6 108) (end 113 108) (width 0.2) (layer F.Cu) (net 15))
 (segment (start 118.6 108) (end 121 108) (width 0.2) (layer F.Cu) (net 17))
 (segment (start 126.6 108) (end 128.4 108) (width 0.2) (layer F.Cu) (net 19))
 (segment (start 128.4 112) (end 128.4 108) (width 0.2) (layer F.Cu) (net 19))
 (segment (start 128.4 112) (end 95.6 112) (width 0.2) (layer F.Cu) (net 19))
 (segment (start 95.6 116) (end 95.6 112) (width 0.2) (layer F.Cu) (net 19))
 (segment (start 95.6 116) (end 97.4 116) (width 0.2) (layer F.Cu) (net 19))
 (segment (start 102.6 116) (end 105 116) (width 0.2) (layer F.Cu) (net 21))
 (segment (start 110.6 116) (end 113 116) (width 0.2) (layer F.Cu) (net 23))
 (segment (start 118.6 116) (end 121 116) (width 0.2) (layer F.Cu) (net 25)))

